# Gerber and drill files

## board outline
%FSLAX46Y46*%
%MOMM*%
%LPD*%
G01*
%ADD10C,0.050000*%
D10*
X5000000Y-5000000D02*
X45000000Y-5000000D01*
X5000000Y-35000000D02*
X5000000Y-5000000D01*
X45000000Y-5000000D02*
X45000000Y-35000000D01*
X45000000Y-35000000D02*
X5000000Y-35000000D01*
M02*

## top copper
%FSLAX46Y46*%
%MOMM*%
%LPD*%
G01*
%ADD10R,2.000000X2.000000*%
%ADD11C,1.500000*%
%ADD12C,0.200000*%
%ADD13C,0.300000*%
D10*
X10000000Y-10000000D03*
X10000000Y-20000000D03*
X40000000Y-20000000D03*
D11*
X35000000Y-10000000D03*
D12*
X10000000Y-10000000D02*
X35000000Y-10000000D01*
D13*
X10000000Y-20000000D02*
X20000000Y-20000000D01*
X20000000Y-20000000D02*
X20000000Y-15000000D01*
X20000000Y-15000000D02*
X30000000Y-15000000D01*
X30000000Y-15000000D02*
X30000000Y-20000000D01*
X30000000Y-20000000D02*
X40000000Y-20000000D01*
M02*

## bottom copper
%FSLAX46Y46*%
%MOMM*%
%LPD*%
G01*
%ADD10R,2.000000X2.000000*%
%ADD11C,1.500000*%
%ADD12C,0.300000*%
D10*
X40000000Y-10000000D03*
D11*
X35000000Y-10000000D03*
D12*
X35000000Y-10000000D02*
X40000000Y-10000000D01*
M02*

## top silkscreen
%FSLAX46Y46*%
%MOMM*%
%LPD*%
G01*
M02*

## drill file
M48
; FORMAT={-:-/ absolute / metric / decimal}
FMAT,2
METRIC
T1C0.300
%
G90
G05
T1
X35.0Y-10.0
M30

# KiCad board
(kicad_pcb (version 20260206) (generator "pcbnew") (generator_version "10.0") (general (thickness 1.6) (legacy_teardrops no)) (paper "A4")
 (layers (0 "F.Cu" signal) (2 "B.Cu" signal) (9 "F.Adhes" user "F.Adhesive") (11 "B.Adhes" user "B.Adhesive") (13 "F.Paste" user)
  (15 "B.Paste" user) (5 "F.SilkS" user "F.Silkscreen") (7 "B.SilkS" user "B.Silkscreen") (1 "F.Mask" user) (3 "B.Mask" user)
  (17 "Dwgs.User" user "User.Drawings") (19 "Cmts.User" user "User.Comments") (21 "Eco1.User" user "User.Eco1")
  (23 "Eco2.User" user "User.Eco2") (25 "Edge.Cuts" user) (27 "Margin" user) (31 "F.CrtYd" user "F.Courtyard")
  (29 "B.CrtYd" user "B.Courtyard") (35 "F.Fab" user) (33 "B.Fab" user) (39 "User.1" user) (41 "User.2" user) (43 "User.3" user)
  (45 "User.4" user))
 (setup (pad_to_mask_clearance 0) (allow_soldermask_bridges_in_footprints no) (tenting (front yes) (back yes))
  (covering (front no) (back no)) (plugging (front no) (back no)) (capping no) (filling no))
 (gr_line (start 5 5) (end 45 5) (stroke (width 0.05) (type default)) (layer "Edge.Cuts"))
 (gr_line (start 5 35) (end 5 5) (stroke (width 0.05) (type default)) (layer "Edge.Cuts"))
 (gr_line (start 45 5) (end 45 35) (stroke (width 0.05) (type default)) (layer "Edge.Cuts"))
 (gr_line (start 45 35) (end 5 35) (stroke (width 0.05) (type default)) (layer "Edge.Cuts"))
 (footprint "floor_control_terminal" (layer "F.Cu") (at 10 10)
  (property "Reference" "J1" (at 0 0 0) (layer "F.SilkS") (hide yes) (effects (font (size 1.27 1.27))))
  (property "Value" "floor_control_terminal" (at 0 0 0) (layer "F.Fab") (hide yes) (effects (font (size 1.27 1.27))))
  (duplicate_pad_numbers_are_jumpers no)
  (pad "1" smd rect (at 0 0) (size 2 2) (layers "F.Cu" "F.Paste" "F.Mask") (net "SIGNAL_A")))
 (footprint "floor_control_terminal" (layer "B.Cu") (at 40 10)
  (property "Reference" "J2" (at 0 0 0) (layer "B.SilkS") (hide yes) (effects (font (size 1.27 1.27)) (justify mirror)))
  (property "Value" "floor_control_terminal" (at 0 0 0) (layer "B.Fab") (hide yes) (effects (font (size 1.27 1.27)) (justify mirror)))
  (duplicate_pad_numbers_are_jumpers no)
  (pad "1" smd rect (at 0 0) (size 2 2) (layers "B.Cu" "B.Paste" "B.Mask") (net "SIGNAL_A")))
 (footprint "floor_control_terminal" (layer "F.Cu") (at 10 20)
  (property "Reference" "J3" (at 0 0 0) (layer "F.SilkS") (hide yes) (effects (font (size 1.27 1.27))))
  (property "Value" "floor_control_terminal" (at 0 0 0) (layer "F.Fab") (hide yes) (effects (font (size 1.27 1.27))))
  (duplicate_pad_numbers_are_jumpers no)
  (pad "1" smd rect (at 0 0) (size 2 2) (layers "F.Cu" "F.Paste" "F.Mask") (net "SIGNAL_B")))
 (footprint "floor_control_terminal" (layer "F.Cu") (at 40 20)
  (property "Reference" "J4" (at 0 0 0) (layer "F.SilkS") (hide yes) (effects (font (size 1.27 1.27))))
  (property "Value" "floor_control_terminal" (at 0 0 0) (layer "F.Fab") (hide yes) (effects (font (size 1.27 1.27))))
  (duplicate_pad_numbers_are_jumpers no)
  (pad "1" smd rect (at 0 0) (size 2 2) (layers "F.Cu" "F.Paste" "F.Mask") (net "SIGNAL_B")))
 (segment (start 10 10) (end 35 10) (width 0.2) (layer "F.Cu") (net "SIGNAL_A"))
 (segment (start 35 10) (end 40 10) (width 0.3) (layer "B.Cu") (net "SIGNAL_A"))
 (via (at 35 10) (size 1.5) (drill 0.3) (layers "F.Cu" "B.Cu") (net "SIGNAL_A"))
 (segment (start 10 20) (end 20 20) (width 0.3) (layer "F.Cu") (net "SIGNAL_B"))
 (segment (start 20 20) (end 20 15) (width 0.3) (layer "F.Cu") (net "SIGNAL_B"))
 (segment (start 20 15) (end 30 15) (width 0.3) (layer "F.Cu") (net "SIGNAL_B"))
 (segment (start 30 15) (end 30 20) (width 0.3) (layer "F.Cu") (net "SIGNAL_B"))
 (segment (start 30 20) (end 40 20) (width 0.3) (layer "F.Cu") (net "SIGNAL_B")))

